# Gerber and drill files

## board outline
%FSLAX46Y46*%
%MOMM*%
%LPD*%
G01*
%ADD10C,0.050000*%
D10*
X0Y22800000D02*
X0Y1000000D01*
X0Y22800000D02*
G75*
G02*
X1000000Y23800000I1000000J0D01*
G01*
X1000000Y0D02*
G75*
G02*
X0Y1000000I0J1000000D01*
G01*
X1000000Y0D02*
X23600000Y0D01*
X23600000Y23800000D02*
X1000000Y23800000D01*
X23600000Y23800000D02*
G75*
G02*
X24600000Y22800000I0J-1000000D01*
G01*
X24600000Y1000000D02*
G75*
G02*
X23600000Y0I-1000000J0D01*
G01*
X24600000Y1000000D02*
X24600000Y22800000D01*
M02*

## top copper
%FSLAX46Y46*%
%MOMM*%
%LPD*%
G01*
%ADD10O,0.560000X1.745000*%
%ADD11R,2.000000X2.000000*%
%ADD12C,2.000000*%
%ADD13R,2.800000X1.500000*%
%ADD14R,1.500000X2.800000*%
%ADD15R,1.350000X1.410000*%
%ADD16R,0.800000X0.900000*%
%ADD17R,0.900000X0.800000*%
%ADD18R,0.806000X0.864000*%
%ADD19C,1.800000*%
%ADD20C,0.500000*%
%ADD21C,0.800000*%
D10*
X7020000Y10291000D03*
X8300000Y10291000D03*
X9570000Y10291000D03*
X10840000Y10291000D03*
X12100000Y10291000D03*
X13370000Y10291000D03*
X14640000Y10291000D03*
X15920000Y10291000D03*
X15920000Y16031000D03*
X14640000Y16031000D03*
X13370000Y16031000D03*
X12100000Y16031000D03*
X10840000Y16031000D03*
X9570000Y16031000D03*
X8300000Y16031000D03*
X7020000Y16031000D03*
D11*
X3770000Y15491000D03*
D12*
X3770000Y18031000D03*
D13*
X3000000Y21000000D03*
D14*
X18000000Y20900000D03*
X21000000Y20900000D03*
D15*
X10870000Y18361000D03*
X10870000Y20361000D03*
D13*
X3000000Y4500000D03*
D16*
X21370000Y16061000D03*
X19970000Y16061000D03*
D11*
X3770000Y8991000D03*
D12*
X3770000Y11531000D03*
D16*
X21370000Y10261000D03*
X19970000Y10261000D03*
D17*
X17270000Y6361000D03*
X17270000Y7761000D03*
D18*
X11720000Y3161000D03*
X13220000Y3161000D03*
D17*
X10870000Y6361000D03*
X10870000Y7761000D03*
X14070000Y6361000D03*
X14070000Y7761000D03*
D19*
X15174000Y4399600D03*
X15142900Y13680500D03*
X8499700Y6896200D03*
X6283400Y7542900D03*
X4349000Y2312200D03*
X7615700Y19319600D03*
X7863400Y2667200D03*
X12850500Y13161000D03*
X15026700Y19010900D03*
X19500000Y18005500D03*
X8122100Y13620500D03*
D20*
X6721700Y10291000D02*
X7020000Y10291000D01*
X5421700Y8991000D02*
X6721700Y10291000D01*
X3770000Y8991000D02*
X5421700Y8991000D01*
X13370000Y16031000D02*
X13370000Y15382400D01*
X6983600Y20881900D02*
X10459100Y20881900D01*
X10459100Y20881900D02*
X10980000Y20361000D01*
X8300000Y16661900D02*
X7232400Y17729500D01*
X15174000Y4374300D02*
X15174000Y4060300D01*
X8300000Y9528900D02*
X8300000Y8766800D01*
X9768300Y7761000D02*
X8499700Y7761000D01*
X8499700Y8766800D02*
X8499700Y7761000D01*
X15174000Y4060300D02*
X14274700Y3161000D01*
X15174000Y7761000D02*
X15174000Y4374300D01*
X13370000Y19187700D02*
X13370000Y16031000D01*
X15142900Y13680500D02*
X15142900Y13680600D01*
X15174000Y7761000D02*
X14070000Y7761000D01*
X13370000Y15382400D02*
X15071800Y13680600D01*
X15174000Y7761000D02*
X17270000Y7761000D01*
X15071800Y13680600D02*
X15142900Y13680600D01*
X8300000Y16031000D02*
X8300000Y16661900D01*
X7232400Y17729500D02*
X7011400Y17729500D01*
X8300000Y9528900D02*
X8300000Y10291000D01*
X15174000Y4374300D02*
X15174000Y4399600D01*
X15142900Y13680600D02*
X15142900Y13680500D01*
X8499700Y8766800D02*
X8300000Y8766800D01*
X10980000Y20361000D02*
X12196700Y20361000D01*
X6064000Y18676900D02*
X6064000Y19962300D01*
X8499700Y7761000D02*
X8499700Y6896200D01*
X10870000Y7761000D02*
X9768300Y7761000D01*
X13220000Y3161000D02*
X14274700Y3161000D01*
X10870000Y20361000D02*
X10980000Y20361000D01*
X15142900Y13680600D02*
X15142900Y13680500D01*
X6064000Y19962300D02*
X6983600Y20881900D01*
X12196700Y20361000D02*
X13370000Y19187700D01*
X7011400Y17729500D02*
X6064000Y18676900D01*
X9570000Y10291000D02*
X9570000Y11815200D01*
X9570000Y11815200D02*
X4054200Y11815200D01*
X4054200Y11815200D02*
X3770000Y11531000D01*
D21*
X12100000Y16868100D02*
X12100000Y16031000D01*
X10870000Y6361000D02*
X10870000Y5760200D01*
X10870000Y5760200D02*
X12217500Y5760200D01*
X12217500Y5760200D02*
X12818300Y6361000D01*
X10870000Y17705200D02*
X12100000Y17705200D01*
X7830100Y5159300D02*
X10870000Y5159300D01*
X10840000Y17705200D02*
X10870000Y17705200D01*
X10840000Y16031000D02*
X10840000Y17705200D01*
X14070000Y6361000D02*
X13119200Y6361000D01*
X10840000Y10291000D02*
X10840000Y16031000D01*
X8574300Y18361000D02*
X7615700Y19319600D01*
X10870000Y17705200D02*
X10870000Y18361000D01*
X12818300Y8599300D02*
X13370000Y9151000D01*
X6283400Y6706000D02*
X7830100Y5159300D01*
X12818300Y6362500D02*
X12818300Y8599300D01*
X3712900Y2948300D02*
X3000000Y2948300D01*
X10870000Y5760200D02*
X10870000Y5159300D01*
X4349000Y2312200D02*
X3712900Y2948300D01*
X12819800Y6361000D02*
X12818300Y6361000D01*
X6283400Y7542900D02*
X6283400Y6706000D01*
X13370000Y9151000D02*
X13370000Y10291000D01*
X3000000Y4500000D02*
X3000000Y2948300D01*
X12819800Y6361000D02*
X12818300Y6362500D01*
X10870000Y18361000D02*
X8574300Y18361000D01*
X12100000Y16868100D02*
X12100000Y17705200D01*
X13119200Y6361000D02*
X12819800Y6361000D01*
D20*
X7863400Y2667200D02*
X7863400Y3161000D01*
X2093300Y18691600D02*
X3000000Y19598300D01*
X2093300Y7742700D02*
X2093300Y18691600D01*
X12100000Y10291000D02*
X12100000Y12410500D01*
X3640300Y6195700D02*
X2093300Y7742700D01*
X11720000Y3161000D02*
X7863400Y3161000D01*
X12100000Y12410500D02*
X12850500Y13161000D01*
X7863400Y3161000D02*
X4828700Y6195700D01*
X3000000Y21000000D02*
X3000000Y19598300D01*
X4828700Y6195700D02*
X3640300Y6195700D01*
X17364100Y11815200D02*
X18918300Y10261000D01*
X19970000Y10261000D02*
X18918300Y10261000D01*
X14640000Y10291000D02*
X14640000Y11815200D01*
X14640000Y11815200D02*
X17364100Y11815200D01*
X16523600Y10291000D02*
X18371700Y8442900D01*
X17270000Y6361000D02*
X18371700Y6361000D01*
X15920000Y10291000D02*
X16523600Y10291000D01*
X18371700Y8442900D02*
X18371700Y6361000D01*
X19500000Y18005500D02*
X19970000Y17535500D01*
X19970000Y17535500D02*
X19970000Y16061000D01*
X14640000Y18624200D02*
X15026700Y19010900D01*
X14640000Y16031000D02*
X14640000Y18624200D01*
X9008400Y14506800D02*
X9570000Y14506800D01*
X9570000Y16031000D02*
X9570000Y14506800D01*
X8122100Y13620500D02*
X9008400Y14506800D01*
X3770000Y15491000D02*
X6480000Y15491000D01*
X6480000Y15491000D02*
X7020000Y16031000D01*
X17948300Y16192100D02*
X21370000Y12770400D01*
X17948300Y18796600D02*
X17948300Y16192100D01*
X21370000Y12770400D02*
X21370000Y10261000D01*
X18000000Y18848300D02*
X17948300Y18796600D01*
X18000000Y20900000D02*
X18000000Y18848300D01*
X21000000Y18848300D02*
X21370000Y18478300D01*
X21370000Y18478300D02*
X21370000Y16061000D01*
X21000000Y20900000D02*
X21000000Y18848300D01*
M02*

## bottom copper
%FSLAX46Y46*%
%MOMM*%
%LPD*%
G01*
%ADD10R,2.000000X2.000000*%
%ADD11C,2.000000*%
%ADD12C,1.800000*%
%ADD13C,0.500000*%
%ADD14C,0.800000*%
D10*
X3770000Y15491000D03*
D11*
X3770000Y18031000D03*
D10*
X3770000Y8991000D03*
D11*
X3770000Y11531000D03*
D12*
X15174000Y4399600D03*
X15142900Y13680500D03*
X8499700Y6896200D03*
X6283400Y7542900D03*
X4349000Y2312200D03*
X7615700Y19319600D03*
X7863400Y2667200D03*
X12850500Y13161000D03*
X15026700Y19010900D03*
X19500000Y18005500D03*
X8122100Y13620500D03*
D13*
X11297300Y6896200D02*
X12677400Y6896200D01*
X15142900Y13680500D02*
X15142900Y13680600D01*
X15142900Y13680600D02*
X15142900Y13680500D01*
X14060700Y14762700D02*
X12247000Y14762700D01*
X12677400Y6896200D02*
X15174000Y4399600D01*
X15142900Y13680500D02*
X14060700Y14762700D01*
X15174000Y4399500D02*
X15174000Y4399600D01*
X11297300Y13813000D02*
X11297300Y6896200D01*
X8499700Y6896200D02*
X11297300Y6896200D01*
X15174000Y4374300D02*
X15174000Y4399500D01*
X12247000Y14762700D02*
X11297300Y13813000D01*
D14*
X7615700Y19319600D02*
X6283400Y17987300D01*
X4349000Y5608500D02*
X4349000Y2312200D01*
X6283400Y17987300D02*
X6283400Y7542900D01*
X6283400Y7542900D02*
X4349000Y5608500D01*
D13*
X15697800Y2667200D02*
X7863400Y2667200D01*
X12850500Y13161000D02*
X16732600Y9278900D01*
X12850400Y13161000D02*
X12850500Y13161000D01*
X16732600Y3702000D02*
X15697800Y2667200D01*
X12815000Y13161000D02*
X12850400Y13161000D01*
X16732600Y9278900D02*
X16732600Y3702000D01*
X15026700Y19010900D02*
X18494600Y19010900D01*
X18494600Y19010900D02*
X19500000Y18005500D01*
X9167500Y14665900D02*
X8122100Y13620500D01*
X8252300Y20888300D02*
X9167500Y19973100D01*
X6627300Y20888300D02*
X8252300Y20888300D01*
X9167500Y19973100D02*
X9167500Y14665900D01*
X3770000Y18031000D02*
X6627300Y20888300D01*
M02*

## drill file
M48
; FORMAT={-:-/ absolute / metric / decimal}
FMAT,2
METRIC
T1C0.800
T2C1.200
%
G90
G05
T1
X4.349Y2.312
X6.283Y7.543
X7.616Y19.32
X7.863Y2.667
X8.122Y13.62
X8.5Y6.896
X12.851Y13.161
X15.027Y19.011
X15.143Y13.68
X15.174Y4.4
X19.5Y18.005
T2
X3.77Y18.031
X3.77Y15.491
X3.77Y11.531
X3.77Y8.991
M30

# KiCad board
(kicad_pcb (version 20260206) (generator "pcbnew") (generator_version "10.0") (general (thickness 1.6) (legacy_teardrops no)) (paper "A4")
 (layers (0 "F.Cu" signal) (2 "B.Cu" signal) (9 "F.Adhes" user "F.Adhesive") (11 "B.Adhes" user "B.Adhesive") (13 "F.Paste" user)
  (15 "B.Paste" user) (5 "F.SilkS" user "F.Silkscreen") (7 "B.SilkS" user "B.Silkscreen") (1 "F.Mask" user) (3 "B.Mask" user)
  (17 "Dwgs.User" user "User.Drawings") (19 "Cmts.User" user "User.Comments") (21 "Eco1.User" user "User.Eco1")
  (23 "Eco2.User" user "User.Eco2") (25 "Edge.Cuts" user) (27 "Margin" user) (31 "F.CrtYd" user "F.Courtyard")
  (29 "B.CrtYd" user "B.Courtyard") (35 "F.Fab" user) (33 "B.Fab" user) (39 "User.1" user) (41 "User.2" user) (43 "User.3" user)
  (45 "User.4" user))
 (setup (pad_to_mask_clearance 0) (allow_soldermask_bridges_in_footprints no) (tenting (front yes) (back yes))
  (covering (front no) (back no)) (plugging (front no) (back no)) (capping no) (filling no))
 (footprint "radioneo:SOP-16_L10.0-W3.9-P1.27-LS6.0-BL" (layer "F.Cu") (at 11.47 -13.161)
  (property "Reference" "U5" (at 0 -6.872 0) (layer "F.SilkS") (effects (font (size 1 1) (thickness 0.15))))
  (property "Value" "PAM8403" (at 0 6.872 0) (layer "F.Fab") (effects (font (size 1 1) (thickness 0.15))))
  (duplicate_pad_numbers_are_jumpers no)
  (pad "1" smd oval (at -4.45 2.87) (size 0.56 1.745) (layers "F.Cu" "F.Mask" "F.Paste") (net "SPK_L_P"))
  (pad "2" smd oval (at -3.17 2.87) (size 0.56 1.745) (layers "F.Cu" "F.Mask" "F.Paste") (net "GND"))
  (pad "3" smd oval (at -1.9 2.87) (size 0.56 1.745) (layers "F.Cu" "F.Mask" "F.Paste") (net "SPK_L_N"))
  (pad "4" smd oval (at -0.63 2.87) (size 0.56 1.745) (layers "F.Cu" "F.Mask" "F.Paste") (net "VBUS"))
  (pad "5" smd oval (at 0.63 2.87) (size 0.56 1.745) (layers "F.Cu" "F.Mask" "F.Paste") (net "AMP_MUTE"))
  (pad "6" smd oval (at 1.9 2.87) (size 0.56 1.745) (layers "F.Cu" "F.Mask" "F.Paste") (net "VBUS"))
  (pad "7" smd oval (at 3.17 2.87) (size 0.56 1.745) (layers "F.Cu" "F.Mask" "F.Paste") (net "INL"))
  (pad "8" smd oval (at 4.45 2.87) (size 0.56 1.745) (layers "F.Cu" "F.Mask" "F.Paste") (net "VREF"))
  (pad "9" smd oval (at 4.45 -2.87) (size 0.56 1.745) (layers "F.Cu" "F.Mask" "F.Paste"))
  (pad "10" smd oval (at 3.17 -2.87) (size 0.56 1.745) (layers "F.Cu" "F.Mask" "F.Paste") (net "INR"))
  (pad "11" smd oval (at 1.9 -2.87) (size 0.56 1.745) (layers "F.Cu" "F.Mask" "F.Paste") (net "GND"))
  (pad "12" smd oval (at 0.63 -2.87) (size 0.56 1.745) (layers "F.Cu" "F.Mask" "F.Paste") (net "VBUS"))
  (pad "13" smd oval (at -0.63 -2.87) (size 0.56 1.745) (layers "F.Cu" "F.Mask" "F.Paste") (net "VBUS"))
  (pad "14" smd oval (at -1.9 -2.87) (size 0.56 1.745) (layers "F.Cu" "F.Mask" "F.Paste") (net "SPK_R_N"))
  (pad "15" smd oval (at -3.17 -2.87) (size 0.56 1.745) (layers "F.Cu" "F.Mask" "F.Paste") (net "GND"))
  (pad "16" smd oval (at -4.45 -2.87) (size 0.56 1.745) (layers "F.Cu" "F.Mask" "F.Paste") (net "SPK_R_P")))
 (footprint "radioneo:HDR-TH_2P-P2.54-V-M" (layer "F.Cu") (at 3.77 -16.761 90)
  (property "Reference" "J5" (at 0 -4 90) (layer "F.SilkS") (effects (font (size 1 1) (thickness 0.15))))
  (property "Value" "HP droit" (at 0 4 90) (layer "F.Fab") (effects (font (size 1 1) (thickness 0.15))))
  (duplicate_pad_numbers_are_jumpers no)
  (pad "1" thru_hole rect (at -1.27 0 90) (size 2 2) (drill 1.199998) (layers "*.Cu" "*.Mask") (remove_unused_layers no) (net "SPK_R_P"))
  (pad "2" thru_hole circle (at 1.27 0 90) (size 2 2) (drill 1.199998) (layers "*.Cu" "*.Mask") (remove_unused_layers no) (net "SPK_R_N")))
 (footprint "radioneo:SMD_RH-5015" (layer "F.Cu") (at 3 -21)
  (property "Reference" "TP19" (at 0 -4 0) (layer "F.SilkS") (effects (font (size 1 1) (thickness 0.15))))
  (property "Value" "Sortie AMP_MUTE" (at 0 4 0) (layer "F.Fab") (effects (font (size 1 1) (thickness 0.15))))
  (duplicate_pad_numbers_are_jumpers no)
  (pad "1" smd rect (at 0 0) (size 2.8 1.5) (layers "F.Cu" "F.Mask" "F.Paste") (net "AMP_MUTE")))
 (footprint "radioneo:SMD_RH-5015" (layer "F.Cu") (at 18 -20.9 90)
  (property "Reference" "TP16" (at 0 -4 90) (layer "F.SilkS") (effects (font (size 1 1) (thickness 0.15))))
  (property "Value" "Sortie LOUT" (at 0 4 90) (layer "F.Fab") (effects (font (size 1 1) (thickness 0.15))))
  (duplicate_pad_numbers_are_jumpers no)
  (pad "1" smd rect (at 0 0 90) (size 2.8 1.5) (layers "F.Cu" "F.Mask" "F.Paste") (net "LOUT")))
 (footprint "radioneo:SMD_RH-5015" (layer "F.Cu") (at 21 -20.9 90)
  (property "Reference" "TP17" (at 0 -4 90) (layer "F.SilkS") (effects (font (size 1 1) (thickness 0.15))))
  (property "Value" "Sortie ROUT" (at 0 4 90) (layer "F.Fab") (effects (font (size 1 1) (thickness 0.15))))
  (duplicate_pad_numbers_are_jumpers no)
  (pad "1" smd rect (at 0 0 90) (size 2.8 1.5) (layers "F.Cu" "F.Mask" "F.Paste") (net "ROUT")))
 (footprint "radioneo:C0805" (layer "F.Cu") (at 10.87 -19.361 90)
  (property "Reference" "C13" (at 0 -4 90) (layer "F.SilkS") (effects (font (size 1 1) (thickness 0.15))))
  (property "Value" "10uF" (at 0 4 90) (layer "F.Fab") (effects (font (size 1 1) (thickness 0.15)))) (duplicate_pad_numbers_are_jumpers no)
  (pad "1" smd rect (at -1 0 90) (size 1.41 1.35) (layers "F.Cu" "F.Mask" "F.Paste") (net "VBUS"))
  (pad "2" smd rect (at 1 0 90) (size 1.41 1.35) (layers "F.Cu" "F.Mask" "F.Paste") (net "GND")))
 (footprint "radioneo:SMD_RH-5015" (layer "F.Cu") (at 3 -4.5)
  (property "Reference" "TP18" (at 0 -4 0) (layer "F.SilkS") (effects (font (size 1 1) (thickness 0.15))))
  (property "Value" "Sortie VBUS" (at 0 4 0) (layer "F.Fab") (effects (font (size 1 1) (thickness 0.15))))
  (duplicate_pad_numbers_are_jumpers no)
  (pad "1" smd rect (at 0 0) (size 2.8 1.5) (layers "F.Cu" "F.Mask" "F.Paste") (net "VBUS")))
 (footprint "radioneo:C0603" (layer "F.Cu") (at 20.67 -16.061 180)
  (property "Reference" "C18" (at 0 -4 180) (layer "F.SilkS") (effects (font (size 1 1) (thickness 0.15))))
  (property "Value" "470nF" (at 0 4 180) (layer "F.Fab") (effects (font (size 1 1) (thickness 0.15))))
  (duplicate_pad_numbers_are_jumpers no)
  (pad "1" smd rect (at -0.7 0 180) (size 0.8 0.9) (layers "F.Cu" "F.Mask" "F.Paste") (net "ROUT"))
  (pad "2" smd rect (at 0.7 0 180) (size 0.8 0.9) (layers "F.Cu" "F.Mask" "F.Paste") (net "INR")))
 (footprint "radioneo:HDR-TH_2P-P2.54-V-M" (layer "F.Cu") (at 3.77 -10.261 90)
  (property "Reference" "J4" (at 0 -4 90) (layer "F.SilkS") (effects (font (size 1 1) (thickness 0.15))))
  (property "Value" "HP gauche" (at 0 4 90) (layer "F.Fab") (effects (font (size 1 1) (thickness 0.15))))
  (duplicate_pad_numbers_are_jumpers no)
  (pad "1" thru_hole rect (at -1.27 0 90) (size 2 2) (drill 1.199998) (layers "*.Cu" "*.Mask") (remove_unused_layers no) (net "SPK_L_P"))
  (pad "2" thru_hole circle (at 1.27 0 90) (size 2 2) (drill 1.199998) (layers "*.Cu" "*.Mask") (remove_unused_layers no) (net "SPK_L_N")))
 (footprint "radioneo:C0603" (layer "F.Cu") (at 20.67 -10.261 180)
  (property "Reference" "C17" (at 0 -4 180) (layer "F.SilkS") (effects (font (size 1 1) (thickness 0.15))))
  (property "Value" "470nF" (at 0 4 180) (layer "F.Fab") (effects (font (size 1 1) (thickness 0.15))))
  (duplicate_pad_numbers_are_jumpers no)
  (pad "1" smd rect (at -0.7 0 180) (size 0.8 0.9) (layers "F.Cu" "F.Mask" "F.Paste") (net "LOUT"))
  (pad "2" smd rect (at 0.7 0 180) (size 0.8 0.9) (layers "F.Cu" "F.Mask" "F.Paste") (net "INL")))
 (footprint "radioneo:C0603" (layer "F.Cu") (at 17.27 -7.061 90)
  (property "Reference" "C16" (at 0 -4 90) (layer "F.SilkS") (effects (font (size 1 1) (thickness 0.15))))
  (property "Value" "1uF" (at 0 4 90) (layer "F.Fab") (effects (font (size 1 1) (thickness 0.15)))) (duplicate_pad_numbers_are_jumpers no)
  (pad "1" smd rect (at -0.7 0 90) (size 0.8 0.9) (layers "F.Cu" "F.Mask" "F.Paste") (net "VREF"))
  (pad "2" smd rect (at 0.7 0 90) (size 0.8 0.9) (layers "F.Cu" "F.Mask" "F.Paste") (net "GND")))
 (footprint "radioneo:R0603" (layer "F.Cu") (at 12.47 -3.161)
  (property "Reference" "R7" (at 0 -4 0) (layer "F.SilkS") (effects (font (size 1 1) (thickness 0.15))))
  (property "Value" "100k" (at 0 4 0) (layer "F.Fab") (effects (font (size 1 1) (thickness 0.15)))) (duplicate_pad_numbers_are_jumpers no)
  (pad "1" smd rect (at -0.75 0) (size 0.806 0.864) (layers "F.Cu" "F.Mask" "F.Paste") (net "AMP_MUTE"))
  (pad "2" smd rect (at 0.75 0) (size 0.806 0.864) (layers "F.Cu" "F.Mask" "F.Paste") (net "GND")))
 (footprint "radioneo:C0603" (layer "F.Cu") (at 10.87 -7.061 90)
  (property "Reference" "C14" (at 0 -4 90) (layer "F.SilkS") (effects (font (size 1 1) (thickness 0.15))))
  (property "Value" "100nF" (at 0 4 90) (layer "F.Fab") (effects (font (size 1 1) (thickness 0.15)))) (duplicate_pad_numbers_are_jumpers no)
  (pad "1" smd rect (at -0.7 0 90) (size 0.8 0.9) (layers "F.Cu" "F.Mask" "F.Paste") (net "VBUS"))
  (pad "2" smd rect (at 0.7 0 90) (size 0.8 0.9) (layers "F.Cu" "F.Mask" "F.Paste") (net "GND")))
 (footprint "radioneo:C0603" (layer "F.Cu") (at 14.07 -7.061 90)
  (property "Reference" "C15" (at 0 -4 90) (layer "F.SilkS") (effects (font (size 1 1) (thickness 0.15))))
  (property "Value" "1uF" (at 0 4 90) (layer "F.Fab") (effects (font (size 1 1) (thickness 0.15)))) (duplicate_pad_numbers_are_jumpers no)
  (pad "1" smd rect (at -0.7 0 90) (size 0.8 0.9) (layers "F.Cu" "F.Mask" "F.Paste") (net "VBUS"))
  (pad "2" smd rect (at 0.7 0 90) (size 0.8 0.9) (layers "F.Cu" "F.Mask" "F.Paste") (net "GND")))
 (gr_line (start 0 -22.8) (end 0 -1) (stroke (width 0.05) (type default)) (layer "Edge.Cuts"))
 (gr_arc (start 0 -22.8) (mid 0.292893 -23.507107) (end 1 -23.8) (stroke (width 0.05) (type default)) (layer "Edge.Cuts"))
 (gr_arc (start 1 0) (mid 0.292893 -0.292893) (end 0 -1) (stroke (width 0.05) (type default)) (layer "Edge.Cuts"))
 (gr_line (start 1 0) (end 23.6 0) (stroke (width 0.05) (type default)) (layer "Edge.Cuts"))
 (gr_line (start 23.6 -23.8) (end 1 -23.8) (stroke (width 0.05) (type default)) (layer "Edge.Cuts"))
 (gr_arc (start 23.6 -23.8) (mid 24.307107 -23.507107) (end 24.6 -22.8) (stroke (width 0.05) (type default)) (layer "Edge.Cuts"))
 (gr_arc (start 24.6 -1) (mid 24.307107 -0.292893) (end 23.6 0) (stroke (width 0.05) (type default)) (layer "Edge.Cuts"))
 (gr_line (start 24.6 -1) (end 24.6 -22.8) (stroke (width 0.05) (type default)) (layer "Edge.Cuts"))
 (segment (start 6.7217 -10.291) (end 7.02 -10.291) (width 0.5) (layer "F.Cu") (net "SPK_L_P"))
 (segment (start 5.4217 -8.991) (end 6.7217 -10.291) (width 0.5) (layer "F.Cu") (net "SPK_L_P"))
 (segment (start 3.77 -8.991) (end 5.4217 -8.991) (width 0.5) (layer "F.Cu") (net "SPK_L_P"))
 (segment (start 13.37 -16.031) (end 13.37 -15.3824) (width 0.5) (layer "F.Cu") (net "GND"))
 (segment (start 6.9836 -20.8819) (end 10.4591 -20.8819) (width 0.5) (layer "F.Cu") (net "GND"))
 (segment (start 10.4591 -20.8819) (end 10.98 -20.361) (width 0.5) (layer "F.Cu") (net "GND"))
 (segment (start 8.3 -16.6619) (end 7.2324 -17.7295) (width 0.5) (layer "F.Cu") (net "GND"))
 (segment (start 15.174 -4.3743) (end 15.174 -4.0603) (width 0.5) (layer "F.Cu") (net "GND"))
 (segment (start 8.3 -9.5289) (end 8.3 -8.7668) (width 0.5) (layer "F.Cu") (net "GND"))
 (segment (start 9.7683 -7.761) (end 8.4997 -7.761) (width 0.5) (layer "F.Cu") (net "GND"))
 (segment (start 8.4997 -8.7668) (end 8.4997 -7.761) (width 0.5) (layer "F.Cu") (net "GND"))
 (segment (start 15.174 -4.0603) (end 14.2747 -3.161) (width 0.5) (layer "F.Cu") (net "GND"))
 (segment (start 15.174 -7.761) (end 15.174 -4.3743) (width 0.5) (layer "F.Cu") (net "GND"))
 (segment (start 13.37 -19.1877) (end 13.37 -16.031) (width 0.5) (layer "F.Cu") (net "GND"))
 (segment (start 15.1429 -13.6805) (end 15.1429 -13.6806) (width 0.5) (layer "F.Cu") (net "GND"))
 (segment (start 15.174 -7.761) (end 14.07 -7.761) (width 0.5) (layer "F.Cu") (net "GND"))
 (segment (start 13.37 -15.3824) (end 15.0718 -13.6806) (width 0.5) (layer "F.Cu") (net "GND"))
 (segment (start 15.174 -7.761) (end 17.27 -7.761) (width 0.5) (layer "F.Cu") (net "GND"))
 (segment (start 15.0718 -13.6806) (end 15.1429 -13.6806) (width 0.5) (layer "F.Cu") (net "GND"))
 (segment (start 8.3 -16.031) (end 8.3 -16.6619) (width 0.5) (layer "F.Cu") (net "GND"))
 (segment (start 7.2324 -17.7295) (end 7.0114 -17.7295) (width 0.5) (layer "F.Cu") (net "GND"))
 (segment (start 8.3 -9.5289) (end 8.3 -10.291) (width 0.5) (layer "F.Cu") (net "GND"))
 (segment (start 15.174 -4.3743) (end 15.174 -4.3996) (width 0.5) (layer "F.Cu") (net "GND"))
 (segment (start 15.1429 -13.6806) (end 15.1429 -13.6805) (width 0.5) (layer "F.Cu") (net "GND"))
 (segment (start 8.4997 -8.7668) (end 8.3 -8.7668) (width 0.5) (layer "F.Cu") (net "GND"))
 (segment (start 10.98 -20.361) (end 12.1967 -20.361) (width 0.5) (layer "F.Cu") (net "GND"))
 (segment (start 6.064 -18.6769) (end 6.064 -19.9623) (width 0.5) (layer "F.Cu") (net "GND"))
 (segment (start 8.4997 -7.761) (end 8.4997 -6.8962) (width 0.5) (layer "F.Cu") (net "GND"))
 (segment (start 10.87 -7.761) (end 9.7683 -7.761) (width 0.5) (layer "F.Cu") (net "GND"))
 (segment (start 13.22 -3.161) (end 14.2747 -3.161) (width 0.5) (layer "F.Cu") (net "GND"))
 (segment (start 10.87 -20.361) (end 10.98 -20.361) (width 0.5) (layer "F.Cu") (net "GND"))
 (segment (start 15.1429 -13.6806) (end 15.1429 -13.6805) (width 0.5) (layer "F.Cu") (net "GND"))
 (segment (start 6.064 -19.9623) (end 6.9836 -20.8819) (width 0.5) (layer "F.Cu") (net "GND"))
 (segment (start 12.1967 -20.361) (end 13.37 -19.1877) (width 0.5) (layer "F.Cu") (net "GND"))
 (segment (start 7.0114 -17.7295) (end 6.064 -18.6769) (width 0.5) (layer "F.Cu") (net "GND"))
 (via (at 15.174 -4.3996) (size 1.8) (drill 0.8) (layers "F.Cu" "B.Cu") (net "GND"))
 (via (at 15.1429 -13.6805) (size 1.8) (drill 0.8) (layers "F.Cu" "B.Cu") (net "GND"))
 (via (at 8.4997 -6.8962) (size 1.8) (drill 0.8) (layers "F.Cu" "B.Cu") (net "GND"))
 (segment (start 11.2973 -6.8962) (end 12.6774 -6.8962) (width 0.5) (layer "B.Cu") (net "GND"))
 (segment (start 15.1429 -13.6805) (end 15.1429 -13.6806) (width 0.5) (layer "B.Cu") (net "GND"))
 (segment (start 15.1429 -13.6806) (end 15.1429 -13.6805) (width 0.5) (layer "B.Cu") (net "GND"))
 (segment (start 14.0607 -14.7627) (end 12.247 -14.7627) (width 0.5) (layer "B.Cu") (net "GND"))
 (segment (start 12.6774 -6.8962) (end 15.174 -4.3996) (width 0.5) (layer "B.Cu") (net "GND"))
 (segment (start 15.1429 -13.6805) (end 14.0607 -14.7627) (width 0.5) (layer "B.Cu") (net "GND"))
 (segment (start 15.174 -4.3995) (end 15.174 -4.3996) (width 0.5) (layer "B.Cu") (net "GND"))
 (segment (start 11.2973 -13.813) (end 11.2973 -6.8962) (width 0.5) (layer "B.Cu") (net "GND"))
 (segment (start 8.4997 -6.8962) (end 11.2973 -6.8962) (width 0.5) (layer "B.Cu") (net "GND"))
 (segment (start 15.174 -4.3743) (end 15.174 -4.3995) (width 0.5) (layer "B.Cu") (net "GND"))
 (segment (start 12.247 -14.7627) (end 11.2973 -13.813) (width 0.5) (layer "B.Cu") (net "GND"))
 (segment (start 9.57 -10.291) (end 9.57 -11.8152) (width 0.5) (layer "F.Cu") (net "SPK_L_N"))
 (segment (start 9.57 -11.8152) (end 4.0542 -11.8152) (width 0.5) (layer "F.Cu") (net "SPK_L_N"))
 (segment (start 4.0542 -11.8152) (end 3.77 -11.531) (width 0.5) (layer "F.Cu") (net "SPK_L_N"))
 (segment (start 12.1 -16.8681) (end 12.1 -16.031) (width 0.8) (layer "F.Cu") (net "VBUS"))
 (segment (start 10.87 -6.361) (end 10.87 -5.7602) (width 0.8) (layer "F.Cu") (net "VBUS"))
 (segment (start 10.87 -5.7602) (end 12.2175 -5.7602) (width 0.8) (layer "F.Cu") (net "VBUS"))
 (segment (start 12.2175 -5.7602) (end 12.8183 -6.361) (width 0.8) (layer "F.Cu") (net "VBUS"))
 (segment (start 10.87 -17.7052) (end 12.1 -17.7052) (width 0.8) (layer "F.Cu") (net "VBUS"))
 (segment (start 7.8301 -5.1593) (end 10.87 -5.1593) (width 0.8) (layer "F.Cu") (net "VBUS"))
 (segment (start 10.84 -17.7052) (end 10.87 -17.7052) (width 0.8) (layer "F.Cu") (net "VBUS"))
 (segment (start 10.84 -16.031) (end 10.84 -17.7052) (width 0.8) (layer "F.Cu") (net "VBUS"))
 (segment (start 14.07 -6.361) (end 13.1192 -6.361) (width 0.8) (layer "F.Cu") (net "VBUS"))
 (segment (start 10.84 -10.291) (end 10.84 -16.031) (width 0.8) (layer "F.Cu") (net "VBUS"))
 (segment (start 8.5743 -18.361) (end 7.6157 -19.3196) (width 0.8) (layer "F.Cu") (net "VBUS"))
 (segment (start 10.87 -17.7052) (end 10.87 -18.361) (width 0.8) (layer "F.Cu") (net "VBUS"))
 (segment (start 12.8183 -8.5993) (end 13.37 -9.151) (width 0.8) (layer "F.Cu") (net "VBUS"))
 (segment (start 6.2834 -6.706) (end 7.8301 -5.1593) (width 0.8) (layer "F.Cu") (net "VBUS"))
 (segment (start 12.8183 -6.3625) (end 12.8183 -8.5993) (width 0.8) (layer "F.Cu") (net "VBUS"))
 (segment (start 3.7129 -2.9483) (end 3 -2.9483) (width 0.8) (layer "F.Cu") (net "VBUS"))
 (segment (start 10.87 -5.7602) (end 10.87 -5.1593) (width 0.8) (layer "F.Cu") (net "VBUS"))
 (segment (start 4.349 -2.3122) (end 3.7129 -2.9483) (width 0.8) (layer "F.Cu") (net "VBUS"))
 (segment (start 12.8198 -6.361) (end 12.8183 -6.361) (width 0.8) (layer "F.Cu") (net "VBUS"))
 (segment (start 6.2834 -7.5429) (end 6.2834 -6.706) (width 0.8) (layer "F.Cu") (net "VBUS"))
 (segment (start 13.37 -9.151) (end 13.37 -10.291) (width 0.8) (layer "F.Cu") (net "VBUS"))
 (segment (start 3 -4.5) (end 3 -2.9483) (width 0.8) (layer "F.Cu") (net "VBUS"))
 (segment (start 12.8198 -6.361) (end 12.8183 -6.3625) (width 0.8) (layer "F.Cu") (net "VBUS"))
 (segment (start 10.87 -18.361) (end 8.5743 -18.361) (width 0.8) (layer "F.Cu") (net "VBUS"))
 (segment (start 12.1 -16.8681) (end 12.1 -17.7052) (width 0.8) (layer "F.Cu") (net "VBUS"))
 (segment (start 13.1192 -6.361) (end 12.8198 -6.361) (width 0.8) (layer "F.Cu") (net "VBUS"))
 (via (at 6.2834 -7.5429) (size 1.8) (drill 0.8) (layers "F.Cu" "B.Cu") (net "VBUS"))
 (via (at 4.349 -2.3122) (size 1.8) (drill 0.8) (layers "F.Cu" "B.Cu") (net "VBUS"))
 (via (at 7.6157 -19.3196) (size 1.8) (drill 0.8) (layers "F.Cu" "B.Cu") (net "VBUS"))
 (segment (start 7.6157 -19.3196) (end 6.2834 -17.9873) (width 0.8) (layer "B.Cu") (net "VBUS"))
 (segment (start 4.349 -5.6085) (end 4.349 -2.3122) (width 0.8) (layer "B.Cu") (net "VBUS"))
 (segment (start 6.2834 -17.9873) (end 6.2834 -7.5429) (width 0.8) (layer "B.Cu") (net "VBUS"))
 (segment (start 6.2834 -7.5429) (end 4.349 -5.6085) (width 0.8) (layer "B.Cu") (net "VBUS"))
 (segment (start 7.8634 -2.6672) (end 7.8634 -3.161) (width 0.5) (layer "F.Cu") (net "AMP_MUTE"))
 (segment (start 2.0933 -18.6916) (end 3 -19.5983) (width 0.5) (layer "F.Cu") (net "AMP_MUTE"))
 (segment (start 2.0933 -7.7427) (end 2.0933 -18.6916) (width 0.5) (layer "F.Cu") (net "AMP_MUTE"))
 (segment (start 12.1 -10.291) (end 12.1 -12.4105) (width 0.5) (layer "F.Cu") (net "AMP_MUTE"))
 (segment (start 3.6403 -6.1957) (end 2.0933 -7.7427) (width 0.5) (layer "F.Cu") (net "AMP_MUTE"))
 (segment (start 11.72 -3.161) (end 7.8634 -3.161) (width 0.5) (layer "F.Cu") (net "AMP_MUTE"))
 (segment (start 12.1 -12.4105) (end 12.8505 -13.161) (width 0.5) (layer "F.Cu") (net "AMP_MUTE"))
 (segment (start 7.8634 -3.161) (end 4.8287 -6.1957) (width 0.5) (layer "F.Cu") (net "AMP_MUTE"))
 (segment (start 3 -21) (end 3 -19.5983) (width 0.5) (layer "F.Cu") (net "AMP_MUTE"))
 (segment (start 4.8287 -6.1957) (end 3.6403 -6.1957) (width 0.5) (layer "F.Cu") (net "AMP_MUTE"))
 (via (at 7.8634 -2.6672) (size 1.8) (drill 0.8) (layers "F.Cu" "B.Cu") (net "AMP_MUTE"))
 (via (at 12.8505 -13.161) (size 1.8) (drill 0.8) (layers "F.Cu" "B.Cu") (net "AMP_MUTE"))
 (segment (start 15.6978 -2.6672) (end 7.8634 -2.6672) (width 0.5) (layer "B.Cu") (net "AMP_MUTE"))
 (segment (start 12.8505 -13.161) (end 16.7326 -9.2789) (width 0.5) (layer "B.Cu") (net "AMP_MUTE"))
 (segment (start 12.8504 -13.161) (end 12.8505 -13.161) (width 0.5) (layer "B.Cu") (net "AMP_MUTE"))
 (segment (start 16.7326 -3.702) (end 15.6978 -2.6672) (width 0.5) (layer "B.Cu") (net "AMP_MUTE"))
 (segment (start 12.815 -13.161) (end 12.8504 -13.161) (width 0.5) (layer "B.Cu") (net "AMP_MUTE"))
 (segment (start 16.7326 -9.2789) (end 16.7326 -3.702) (width 0.5) (layer "B.Cu") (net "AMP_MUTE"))
 (segment (start 17.3641 -11.8152) (end 18.9183 -10.261) (width 0.5) (layer "F.Cu") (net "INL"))
 (segment (start 19.97 -10.261) (end 18.9183 -10.261) (width 0.5) (layer "F.Cu") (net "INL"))
 (segment (start 14.64 -10.291) (end 14.64 -11.8152) (width 0.5) (layer "F.Cu") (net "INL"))
 (segment (start 14.64 -11.8152) (end 17.3641 -11.8152) (width 0.5) (layer "F.Cu") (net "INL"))
 (segment (start 16.5236 -10.291) (end 18.3717 -8.4429) (width 0.5) (layer "F.Cu") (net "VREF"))
 (segment (start 17.27 -6.361) (end 18.3717 -6.361) (width 0.5) (layer "F.Cu") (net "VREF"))
 (segment (start 15.92 -10.291) (end 16.5236 -10.291) (width 0.5) (layer "F.Cu") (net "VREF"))
 (segment (start 18.3717 -8.4429) (end 18.3717 -6.361) (width 0.5) (layer "F.Cu") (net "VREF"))
 (segment (start 19.5 -18.0055) (end 19.97 -17.5355) (width 0.5) (layer "F.Cu") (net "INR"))
 (segment (start 19.97 -17.5355) (end 19.97 -16.061) (width 0.5) (layer "F.Cu") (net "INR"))
 (segment (start 14.64 -18.6242) (end 15.0267 -19.0109) (width 0.5) (layer "F.Cu") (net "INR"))
 (segment (start 14.64 -16.031) (end 14.64 -18.6242) (width 0.5) (layer "F.Cu") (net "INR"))
 (via (at 15.0267 -19.0109) (size 1.8) (drill 0.8) (layers "F.Cu" "B.Cu") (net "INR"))
 (via (at 19.5 -18.0055) (size 1.8) (drill 0.8) (layers "F.Cu" "B.Cu") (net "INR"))
 (segment (start 15.0267 -19.0109) (end 18.4946 -19.0109) (width 0.5) (layer "B.Cu") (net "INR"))
 (segment (start 18.4946 -19.0109) (end 19.5 -18.0055) (width 0.5) (layer "B.Cu") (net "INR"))
 (segment (start 9.0084 -14.5068) (end 9.57 -14.5068) (width 0.5) (layer "F.Cu") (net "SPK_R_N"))
 (segment (start 9.57 -16.031) (end 9.57 -14.5068) (width 0.5) (layer "F.Cu") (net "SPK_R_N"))
 (segment (start 8.1221 -13.6205) (end 9.0084 -14.5068) (width 0.5) (layer "F.Cu") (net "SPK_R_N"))
 (via (at 8.1221 -13.6205) (size 1.8) (drill 0.8) (layers "F.Cu" "B.Cu") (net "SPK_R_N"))
 (segment (start 9.1675 -14.6659) (end 8.1221 -13.6205) (width 0.5) (layer "B.Cu") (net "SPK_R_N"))
 (segment (start 8.2523 -20.8883) (end 9.1675 -19.9731) (width 0.5) (layer "B.Cu") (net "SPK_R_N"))
 (segment (start 6.6273 -20.8883) (end 8.2523 -20.8883) (width 0.5) (layer "B.Cu") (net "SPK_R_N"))
 (segment (start 9.1675 -19.9731) (end 9.1675 -14.6659) (width 0.5) (layer "B.Cu") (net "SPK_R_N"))
 (segment (start 3.77 -18.031) (end 6.6273 -20.8883) (width 0.5) (layer "B.Cu") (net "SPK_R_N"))
 (segment (start 3.77 -15.491) (end 6.48 -15.491) (width 0.5) (layer "F.Cu") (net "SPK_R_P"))
 (segment (start 6.48 -15.491) (end 7.02 -16.031) (width 0.5) (layer "F.Cu") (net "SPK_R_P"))
 (segment (start 17.9483 -16.1921) (end 21.37 -12.7704) (width 0.5) (layer "F.Cu") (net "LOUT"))
 (segment (start 17.9483 -18.7966) (end 17.9483 -16.1921) (width 0.5) (layer "F.Cu") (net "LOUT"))
 (segment (start 21.37 -12.7704) (end 21.37 -10.261) (width 0.5) (layer "F.Cu") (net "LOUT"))
 (segment (start 18 -18.8483) (end 17.9483 -18.7966) (width 0.5) (layer "F.Cu") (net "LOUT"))
 (segment (start 18 -20.9) (end 18 -18.8483) (width 0.5) (layer "F.Cu") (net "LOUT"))
 (segment (start 21 -18.8483) (end 21.37 -18.4783) (width 0.5) (layer "F.Cu") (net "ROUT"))
 (segment (start 21.37 -18.4783) (end 21.37 -16.061) (width 0.5) (layer "F.Cu") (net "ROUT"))
 (segment (start 21 -20.9) (end 21 -18.8483) (width 0.5) (layer "F.Cu") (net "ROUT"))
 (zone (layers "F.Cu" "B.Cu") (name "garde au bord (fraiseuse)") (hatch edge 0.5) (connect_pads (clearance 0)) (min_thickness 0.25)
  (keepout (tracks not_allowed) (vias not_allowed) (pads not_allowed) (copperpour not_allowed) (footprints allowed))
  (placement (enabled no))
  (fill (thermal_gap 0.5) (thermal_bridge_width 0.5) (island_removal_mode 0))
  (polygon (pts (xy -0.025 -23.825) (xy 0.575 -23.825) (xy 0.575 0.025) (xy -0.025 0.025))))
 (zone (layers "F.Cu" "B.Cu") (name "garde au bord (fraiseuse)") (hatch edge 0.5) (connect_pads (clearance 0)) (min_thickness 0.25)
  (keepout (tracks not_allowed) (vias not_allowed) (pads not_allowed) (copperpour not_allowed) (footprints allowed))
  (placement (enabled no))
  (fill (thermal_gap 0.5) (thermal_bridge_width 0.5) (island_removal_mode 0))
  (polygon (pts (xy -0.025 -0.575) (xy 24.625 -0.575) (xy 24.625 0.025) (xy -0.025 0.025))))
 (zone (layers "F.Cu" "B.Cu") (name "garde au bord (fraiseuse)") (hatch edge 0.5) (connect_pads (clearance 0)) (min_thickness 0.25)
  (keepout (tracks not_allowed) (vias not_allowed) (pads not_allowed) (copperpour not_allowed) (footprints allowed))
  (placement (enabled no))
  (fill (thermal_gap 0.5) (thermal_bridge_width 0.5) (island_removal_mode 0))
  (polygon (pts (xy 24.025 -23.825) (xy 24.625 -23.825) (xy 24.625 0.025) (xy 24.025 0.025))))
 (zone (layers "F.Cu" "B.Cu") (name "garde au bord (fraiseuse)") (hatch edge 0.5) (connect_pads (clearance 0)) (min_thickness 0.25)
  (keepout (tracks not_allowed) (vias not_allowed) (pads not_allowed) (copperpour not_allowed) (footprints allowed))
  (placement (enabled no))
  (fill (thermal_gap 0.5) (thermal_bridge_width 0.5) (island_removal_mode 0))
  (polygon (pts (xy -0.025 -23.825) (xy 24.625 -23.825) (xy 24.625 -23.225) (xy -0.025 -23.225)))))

